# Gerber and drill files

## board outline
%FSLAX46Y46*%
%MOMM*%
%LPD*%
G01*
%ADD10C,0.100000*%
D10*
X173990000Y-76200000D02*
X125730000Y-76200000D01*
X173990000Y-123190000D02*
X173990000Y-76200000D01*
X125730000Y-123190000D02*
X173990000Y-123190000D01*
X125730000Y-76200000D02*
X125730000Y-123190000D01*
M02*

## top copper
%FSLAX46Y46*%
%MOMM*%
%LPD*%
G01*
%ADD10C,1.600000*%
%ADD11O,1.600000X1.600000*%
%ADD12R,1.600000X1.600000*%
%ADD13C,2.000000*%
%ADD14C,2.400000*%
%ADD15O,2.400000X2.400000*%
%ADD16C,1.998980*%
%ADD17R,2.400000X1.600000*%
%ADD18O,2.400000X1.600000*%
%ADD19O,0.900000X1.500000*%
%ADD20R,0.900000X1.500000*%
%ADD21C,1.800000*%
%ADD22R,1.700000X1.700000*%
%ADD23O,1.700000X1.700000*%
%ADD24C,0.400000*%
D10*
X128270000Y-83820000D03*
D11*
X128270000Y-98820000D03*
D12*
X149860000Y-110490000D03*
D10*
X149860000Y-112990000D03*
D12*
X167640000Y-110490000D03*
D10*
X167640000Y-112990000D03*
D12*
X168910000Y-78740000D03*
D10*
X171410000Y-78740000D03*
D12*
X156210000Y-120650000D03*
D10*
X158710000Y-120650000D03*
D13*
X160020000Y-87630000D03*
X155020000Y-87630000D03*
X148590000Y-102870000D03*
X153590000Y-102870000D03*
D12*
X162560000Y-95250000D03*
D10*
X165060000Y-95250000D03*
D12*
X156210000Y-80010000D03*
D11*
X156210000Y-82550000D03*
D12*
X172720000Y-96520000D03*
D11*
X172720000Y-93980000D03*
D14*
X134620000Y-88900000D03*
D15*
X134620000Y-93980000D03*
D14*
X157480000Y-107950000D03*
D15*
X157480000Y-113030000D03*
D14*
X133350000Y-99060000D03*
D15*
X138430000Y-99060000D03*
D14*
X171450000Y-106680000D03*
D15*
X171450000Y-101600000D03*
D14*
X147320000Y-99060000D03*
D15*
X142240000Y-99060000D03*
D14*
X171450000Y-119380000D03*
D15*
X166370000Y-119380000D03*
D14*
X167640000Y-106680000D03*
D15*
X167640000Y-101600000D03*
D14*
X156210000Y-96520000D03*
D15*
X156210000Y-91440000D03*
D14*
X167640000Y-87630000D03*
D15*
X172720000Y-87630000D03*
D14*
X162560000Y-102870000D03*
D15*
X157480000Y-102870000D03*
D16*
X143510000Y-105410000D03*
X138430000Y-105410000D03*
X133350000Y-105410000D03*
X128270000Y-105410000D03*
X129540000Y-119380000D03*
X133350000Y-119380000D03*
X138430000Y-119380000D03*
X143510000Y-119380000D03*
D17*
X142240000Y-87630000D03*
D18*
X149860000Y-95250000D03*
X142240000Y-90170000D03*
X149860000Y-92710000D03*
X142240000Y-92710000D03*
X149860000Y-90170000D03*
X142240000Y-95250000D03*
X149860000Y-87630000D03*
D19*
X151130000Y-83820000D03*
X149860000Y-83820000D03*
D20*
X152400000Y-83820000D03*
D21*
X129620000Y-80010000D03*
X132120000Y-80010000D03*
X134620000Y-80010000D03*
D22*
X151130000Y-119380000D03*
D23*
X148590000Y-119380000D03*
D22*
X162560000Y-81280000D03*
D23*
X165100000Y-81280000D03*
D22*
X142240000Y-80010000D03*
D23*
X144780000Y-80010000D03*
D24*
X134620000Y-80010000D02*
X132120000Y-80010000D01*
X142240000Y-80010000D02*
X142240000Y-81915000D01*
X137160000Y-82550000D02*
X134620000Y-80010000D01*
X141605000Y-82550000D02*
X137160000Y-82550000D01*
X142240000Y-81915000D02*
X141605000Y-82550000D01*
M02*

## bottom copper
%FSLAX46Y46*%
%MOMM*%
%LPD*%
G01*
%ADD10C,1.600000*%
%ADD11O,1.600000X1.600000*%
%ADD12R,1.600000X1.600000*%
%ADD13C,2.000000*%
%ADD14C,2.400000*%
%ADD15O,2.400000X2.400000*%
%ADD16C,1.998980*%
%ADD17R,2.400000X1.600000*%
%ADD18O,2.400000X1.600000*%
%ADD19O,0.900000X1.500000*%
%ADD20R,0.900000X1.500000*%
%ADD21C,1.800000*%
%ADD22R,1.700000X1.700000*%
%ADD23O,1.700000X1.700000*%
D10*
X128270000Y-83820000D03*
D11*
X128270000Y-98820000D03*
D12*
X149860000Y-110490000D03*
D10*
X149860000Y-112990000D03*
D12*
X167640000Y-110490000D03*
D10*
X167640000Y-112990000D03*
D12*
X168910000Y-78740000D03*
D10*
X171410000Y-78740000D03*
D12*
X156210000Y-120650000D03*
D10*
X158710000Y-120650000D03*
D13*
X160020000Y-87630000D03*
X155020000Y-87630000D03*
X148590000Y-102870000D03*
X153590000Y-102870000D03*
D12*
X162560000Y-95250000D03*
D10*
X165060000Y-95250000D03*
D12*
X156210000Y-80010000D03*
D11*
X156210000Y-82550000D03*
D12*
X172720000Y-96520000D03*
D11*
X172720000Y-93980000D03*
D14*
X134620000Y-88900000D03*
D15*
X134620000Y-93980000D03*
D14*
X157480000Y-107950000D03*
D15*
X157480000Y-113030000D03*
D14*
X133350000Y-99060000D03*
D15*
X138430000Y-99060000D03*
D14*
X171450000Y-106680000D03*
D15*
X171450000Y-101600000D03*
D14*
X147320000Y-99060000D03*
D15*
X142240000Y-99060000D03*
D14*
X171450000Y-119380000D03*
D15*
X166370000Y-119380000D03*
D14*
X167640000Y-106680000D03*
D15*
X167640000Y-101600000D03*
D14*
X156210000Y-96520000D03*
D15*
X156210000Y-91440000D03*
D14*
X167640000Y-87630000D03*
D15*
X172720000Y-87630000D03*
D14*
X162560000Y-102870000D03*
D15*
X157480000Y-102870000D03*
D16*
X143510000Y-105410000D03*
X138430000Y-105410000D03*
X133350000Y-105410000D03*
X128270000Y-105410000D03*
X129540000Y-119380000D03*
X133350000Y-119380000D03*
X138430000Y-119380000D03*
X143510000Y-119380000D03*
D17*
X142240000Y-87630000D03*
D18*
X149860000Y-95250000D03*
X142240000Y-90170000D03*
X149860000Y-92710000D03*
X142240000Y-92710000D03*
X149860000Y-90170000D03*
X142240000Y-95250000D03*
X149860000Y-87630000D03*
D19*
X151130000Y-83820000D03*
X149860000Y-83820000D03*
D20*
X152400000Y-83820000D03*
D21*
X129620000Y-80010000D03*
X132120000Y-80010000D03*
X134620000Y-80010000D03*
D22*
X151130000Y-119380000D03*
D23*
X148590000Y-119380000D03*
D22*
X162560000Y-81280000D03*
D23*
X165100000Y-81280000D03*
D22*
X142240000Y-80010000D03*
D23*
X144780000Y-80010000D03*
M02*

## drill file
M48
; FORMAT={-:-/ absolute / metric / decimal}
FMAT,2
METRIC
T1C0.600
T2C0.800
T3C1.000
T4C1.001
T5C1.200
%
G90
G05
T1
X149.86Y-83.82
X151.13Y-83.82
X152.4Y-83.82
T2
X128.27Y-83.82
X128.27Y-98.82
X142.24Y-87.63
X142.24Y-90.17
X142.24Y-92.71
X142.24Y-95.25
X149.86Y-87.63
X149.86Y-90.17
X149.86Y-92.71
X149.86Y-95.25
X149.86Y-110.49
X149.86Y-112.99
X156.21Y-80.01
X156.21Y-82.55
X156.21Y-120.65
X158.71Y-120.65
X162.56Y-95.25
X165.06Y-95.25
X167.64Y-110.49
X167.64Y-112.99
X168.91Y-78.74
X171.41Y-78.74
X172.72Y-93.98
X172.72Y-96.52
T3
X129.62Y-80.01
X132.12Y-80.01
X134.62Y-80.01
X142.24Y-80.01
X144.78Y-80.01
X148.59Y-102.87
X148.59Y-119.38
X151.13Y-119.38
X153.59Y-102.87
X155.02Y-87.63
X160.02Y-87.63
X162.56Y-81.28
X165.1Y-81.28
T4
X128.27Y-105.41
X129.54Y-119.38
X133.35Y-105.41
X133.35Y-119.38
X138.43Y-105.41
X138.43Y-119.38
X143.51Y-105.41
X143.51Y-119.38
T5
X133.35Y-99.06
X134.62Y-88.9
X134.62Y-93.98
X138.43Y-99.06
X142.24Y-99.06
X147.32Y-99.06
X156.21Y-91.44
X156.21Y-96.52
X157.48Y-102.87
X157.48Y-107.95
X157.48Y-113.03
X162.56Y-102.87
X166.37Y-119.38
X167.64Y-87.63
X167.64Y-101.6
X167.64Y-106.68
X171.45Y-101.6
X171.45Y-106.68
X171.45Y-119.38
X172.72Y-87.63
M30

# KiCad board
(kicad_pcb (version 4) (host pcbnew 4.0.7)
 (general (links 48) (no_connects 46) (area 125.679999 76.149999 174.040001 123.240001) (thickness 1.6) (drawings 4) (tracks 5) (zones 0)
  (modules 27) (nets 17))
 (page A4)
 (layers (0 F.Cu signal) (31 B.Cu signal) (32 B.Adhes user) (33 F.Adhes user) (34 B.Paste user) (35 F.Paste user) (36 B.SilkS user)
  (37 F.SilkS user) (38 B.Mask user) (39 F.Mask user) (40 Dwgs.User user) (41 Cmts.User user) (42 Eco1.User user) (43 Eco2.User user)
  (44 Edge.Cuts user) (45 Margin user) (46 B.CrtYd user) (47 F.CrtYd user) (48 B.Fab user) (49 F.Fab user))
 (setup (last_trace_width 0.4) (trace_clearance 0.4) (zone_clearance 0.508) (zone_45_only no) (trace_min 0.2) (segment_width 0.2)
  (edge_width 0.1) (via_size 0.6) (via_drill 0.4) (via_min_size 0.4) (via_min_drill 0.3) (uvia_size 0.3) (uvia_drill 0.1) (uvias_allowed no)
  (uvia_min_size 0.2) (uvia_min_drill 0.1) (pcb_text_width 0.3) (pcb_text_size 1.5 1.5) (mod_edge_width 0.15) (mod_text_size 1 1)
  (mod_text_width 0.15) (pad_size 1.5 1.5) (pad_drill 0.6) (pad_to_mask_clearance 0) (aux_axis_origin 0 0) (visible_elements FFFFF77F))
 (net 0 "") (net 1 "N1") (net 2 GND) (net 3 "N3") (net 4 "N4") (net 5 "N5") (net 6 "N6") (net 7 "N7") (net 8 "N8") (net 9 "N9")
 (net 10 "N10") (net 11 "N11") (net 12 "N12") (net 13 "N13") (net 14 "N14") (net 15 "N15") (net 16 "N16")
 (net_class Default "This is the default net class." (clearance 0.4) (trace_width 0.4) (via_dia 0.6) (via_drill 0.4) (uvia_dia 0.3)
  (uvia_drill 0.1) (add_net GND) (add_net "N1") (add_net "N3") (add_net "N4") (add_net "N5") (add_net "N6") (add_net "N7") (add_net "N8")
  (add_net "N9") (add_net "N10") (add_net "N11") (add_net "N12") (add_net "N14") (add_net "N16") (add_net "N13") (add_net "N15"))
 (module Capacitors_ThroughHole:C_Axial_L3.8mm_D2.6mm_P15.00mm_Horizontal (layer F.Cu) (at 128.27 83.82 270)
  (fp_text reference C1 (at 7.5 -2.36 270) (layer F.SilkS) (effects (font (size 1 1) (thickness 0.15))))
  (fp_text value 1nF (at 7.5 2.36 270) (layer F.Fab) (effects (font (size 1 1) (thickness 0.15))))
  (pad 1 thru_hole circle (at 0 0 270) (size 1.6 1.6) (drill 0.8) (layers *.Cu *.Mask) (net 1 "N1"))
  (pad 2 thru_hole oval (at 15 0 270) (size 1.6 1.6) (drill 0.8) (layers *.Cu *.Mask) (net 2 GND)))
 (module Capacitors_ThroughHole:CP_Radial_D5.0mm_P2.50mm (layer F.Cu) (at 149.86 110.49 270)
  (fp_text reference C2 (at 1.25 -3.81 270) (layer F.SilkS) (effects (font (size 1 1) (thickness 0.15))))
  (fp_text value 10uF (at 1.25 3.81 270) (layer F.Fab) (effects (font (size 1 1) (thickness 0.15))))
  (pad 1 thru_hole rect (at 0 0 270) (size 1.6 1.6) (drill 0.8) (layers *.Cu *.Mask) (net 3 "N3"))
  (pad 2 thru_hole circle (at 2.5 0 270) (size 1.6 1.6) (drill 0.8) (layers *.Cu *.Mask) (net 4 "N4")))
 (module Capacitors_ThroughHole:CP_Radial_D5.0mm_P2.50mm (layer F.Cu) (at 167.64 110.49 270)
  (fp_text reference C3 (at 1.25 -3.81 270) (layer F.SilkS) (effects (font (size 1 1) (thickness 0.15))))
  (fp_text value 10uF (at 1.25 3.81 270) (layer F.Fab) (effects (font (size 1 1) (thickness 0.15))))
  (pad 1 thru_hole rect (at 0 0 270) (size 1.6 1.6) (drill 0.8) (layers *.Cu *.Mask) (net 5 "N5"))
  (pad 2 thru_hole circle (at 2.5 0 270) (size 1.6 1.6) (drill 0.8) (layers *.Cu *.Mask) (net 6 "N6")))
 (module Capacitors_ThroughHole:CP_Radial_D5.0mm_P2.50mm (layer F.Cu) (at 168.91 78.74)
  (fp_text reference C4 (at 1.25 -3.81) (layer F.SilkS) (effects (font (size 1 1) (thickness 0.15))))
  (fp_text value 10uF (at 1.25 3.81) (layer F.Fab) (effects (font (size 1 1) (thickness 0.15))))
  (pad 1 thru_hole rect (at 0 0) (size 1.6 1.6) (drill 0.8) (layers *.Cu *.Mask) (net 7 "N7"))
  (pad 2 thru_hole circle (at 2.5 0) (size 1.6 1.6) (drill 0.8) (layers *.Cu *.Mask) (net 2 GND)))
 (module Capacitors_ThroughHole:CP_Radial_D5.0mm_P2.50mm (layer F.Cu) (at 156.21 120.65)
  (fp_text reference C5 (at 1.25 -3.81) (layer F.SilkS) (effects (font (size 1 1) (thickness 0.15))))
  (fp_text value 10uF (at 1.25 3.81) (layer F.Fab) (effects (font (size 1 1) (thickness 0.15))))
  (pad 1 thru_hole rect (at 0 0) (size 1.6 1.6) (drill 0.8) (layers *.Cu *.Mask) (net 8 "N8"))
  (pad 2 thru_hole circle (at 2.5 0) (size 1.6 1.6) (drill 0.8) (layers *.Cu *.Mask) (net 2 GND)))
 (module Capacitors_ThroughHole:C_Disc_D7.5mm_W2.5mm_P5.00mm (layer F.Cu) (at 160.02 87.63 180)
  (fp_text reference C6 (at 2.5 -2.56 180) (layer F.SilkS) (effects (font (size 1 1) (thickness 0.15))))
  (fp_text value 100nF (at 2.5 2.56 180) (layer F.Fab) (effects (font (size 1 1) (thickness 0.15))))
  (pad 1 thru_hole circle (at 0 0 180) (size 2 2) (drill 1) (layers *.Cu *.Mask) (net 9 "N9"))
  (pad 2 thru_hole circle (at 5 0 180) (size 2 2) (drill 1) (layers *.Cu *.Mask) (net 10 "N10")))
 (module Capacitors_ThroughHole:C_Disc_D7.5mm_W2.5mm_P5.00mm (layer F.Cu) (at 148.59 102.87)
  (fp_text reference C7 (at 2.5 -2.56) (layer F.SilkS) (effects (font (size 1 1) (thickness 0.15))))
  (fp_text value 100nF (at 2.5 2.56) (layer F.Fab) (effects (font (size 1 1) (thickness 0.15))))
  (pad 1 thru_hole circle (at 0 0) (size 2 2) (drill 1) (layers *.Cu *.Mask) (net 2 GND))
  (pad 2 thru_hole circle (at 5 0) (size 2 2) (drill 1) (layers *.Cu *.Mask) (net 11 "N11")))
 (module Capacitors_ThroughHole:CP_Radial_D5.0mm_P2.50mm (layer F.Cu) (at 162.56 95.25)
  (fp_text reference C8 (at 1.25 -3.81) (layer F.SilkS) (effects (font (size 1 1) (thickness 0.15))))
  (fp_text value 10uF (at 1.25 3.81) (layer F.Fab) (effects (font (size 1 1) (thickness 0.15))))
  (pad 1 thru_hole rect (at 0 0) (size 1.6 1.6) (drill 0.8) (layers *.Cu *.Mask) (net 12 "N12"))
  (pad 2 thru_hole circle (at 2.5 0) (size 1.6 1.6) (drill 0.8) (layers *.Cu *.Mask) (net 2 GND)))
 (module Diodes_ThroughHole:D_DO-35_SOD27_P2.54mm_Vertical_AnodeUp (layer F.Cu) (at 156.21 80.01 270)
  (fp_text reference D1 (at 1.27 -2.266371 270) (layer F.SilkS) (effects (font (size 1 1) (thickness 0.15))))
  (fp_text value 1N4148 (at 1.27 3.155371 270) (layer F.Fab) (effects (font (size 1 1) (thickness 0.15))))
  (pad 1 thru_hole rect (at 0 0 270) (size 1.6 1.6) (drill 0.8) (layers *.Cu *.Mask) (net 9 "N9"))
  (pad 2 thru_hole oval (at 2.54 0 270) (size 1.6 1.6) (drill 0.8) (layers *.Cu *.Mask) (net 2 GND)))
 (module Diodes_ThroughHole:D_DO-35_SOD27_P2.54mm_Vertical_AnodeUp (layer F.Cu) (at 172.72 96.52 90)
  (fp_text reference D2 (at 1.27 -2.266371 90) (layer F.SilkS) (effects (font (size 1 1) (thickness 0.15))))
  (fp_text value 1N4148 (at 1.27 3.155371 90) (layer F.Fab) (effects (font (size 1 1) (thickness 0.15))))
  (pad 1 thru_hole rect (at 0 0 90) (size 1.6 1.6) (drill 0.8) (layers *.Cu *.Mask) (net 11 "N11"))
  (pad 2 thru_hole oval (at 2.54 0 90) (size 1.6 1.6) (drill 0.8) (layers *.Cu *.Mask) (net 9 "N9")))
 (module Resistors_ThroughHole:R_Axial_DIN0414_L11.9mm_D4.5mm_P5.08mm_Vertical (layer F.Cu) (at 134.62 88.9 270)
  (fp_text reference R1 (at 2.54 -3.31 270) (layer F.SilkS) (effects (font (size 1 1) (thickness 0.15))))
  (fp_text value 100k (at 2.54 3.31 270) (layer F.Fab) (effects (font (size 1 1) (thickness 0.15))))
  (pad 1 thru_hole circle (at 0 0 270) (size 2.4 2.4) (drill 1.2) (layers *.Cu *.Mask) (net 8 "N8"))
  (pad 2 thru_hole oval (at 5.08 0 270) (size 2.4 2.4) (drill 1.2) (layers *.Cu *.Mask) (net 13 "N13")))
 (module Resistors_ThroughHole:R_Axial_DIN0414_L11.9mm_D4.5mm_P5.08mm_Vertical (layer F.Cu) (at 157.48 107.95 270)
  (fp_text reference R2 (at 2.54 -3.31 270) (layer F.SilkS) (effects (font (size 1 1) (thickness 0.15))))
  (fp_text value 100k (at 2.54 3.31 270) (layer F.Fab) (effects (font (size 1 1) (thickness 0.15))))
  (pad 1 thru_hole circle (at 0 0 270) (size 2.4 2.4) (drill 1.2) (layers *.Cu *.Mask) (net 13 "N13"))
  (pad 2 thru_hole oval (at 5.08 0 270) (size 2.4 2.4) (drill 1.2) (layers *.Cu *.Mask) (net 2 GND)))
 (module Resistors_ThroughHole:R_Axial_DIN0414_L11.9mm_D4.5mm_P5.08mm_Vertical (layer F.Cu) (at 133.35 99.06)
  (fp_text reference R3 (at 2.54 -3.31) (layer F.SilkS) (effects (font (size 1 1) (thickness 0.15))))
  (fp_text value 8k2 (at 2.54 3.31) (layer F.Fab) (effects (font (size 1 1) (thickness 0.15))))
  (pad 1 thru_hole circle (at 0 0) (size 2.4 2.4) (drill 1.2) (layers *.Cu *.Mask) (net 3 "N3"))
  (pad 2 thru_hole oval (at 5.08 0) (size 2.4 2.4) (drill 1.2) (layers *.Cu *.Mask) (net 1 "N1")))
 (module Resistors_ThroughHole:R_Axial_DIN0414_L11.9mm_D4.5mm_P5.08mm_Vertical (layer F.Cu) (at 171.45 106.68 90)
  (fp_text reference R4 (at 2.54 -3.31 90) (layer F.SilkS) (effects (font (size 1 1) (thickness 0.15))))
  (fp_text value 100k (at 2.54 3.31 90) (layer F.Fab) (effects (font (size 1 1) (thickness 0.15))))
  (pad 1 thru_hole circle (at 0 0 90) (size 2.4 2.4) (drill 1.2) (layers *.Cu *.Mask) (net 3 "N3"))
  (pad 2 thru_hole oval (at 5.08 0 90) (size 2.4 2.4) (drill 1.2) (layers *.Cu *.Mask) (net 13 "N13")))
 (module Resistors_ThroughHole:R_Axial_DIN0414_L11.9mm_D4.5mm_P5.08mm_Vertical (layer F.Cu) (at 147.32 99.06 180)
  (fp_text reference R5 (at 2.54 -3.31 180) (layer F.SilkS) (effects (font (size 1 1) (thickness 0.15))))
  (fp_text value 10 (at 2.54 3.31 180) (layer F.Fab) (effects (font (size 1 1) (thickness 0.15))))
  (pad 1 thru_hole circle (at 0 0 180) (size 2.4 2.4) (drill 1.2) (layers *.Cu *.Mask) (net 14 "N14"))
  (pad 2 thru_hole oval (at 5.08 0 180) (size 2.4 2.4) (drill 1.2) (layers *.Cu *.Mask) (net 2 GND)))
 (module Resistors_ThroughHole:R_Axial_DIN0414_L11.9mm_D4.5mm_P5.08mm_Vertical (layer F.Cu) (at 171.45 119.38 180)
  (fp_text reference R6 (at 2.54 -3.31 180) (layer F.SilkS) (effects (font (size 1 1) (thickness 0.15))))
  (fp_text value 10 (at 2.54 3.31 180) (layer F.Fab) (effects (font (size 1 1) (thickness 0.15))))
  (pad 1 thru_hole circle (at 0 0 180) (size 2.4 2.4) (drill 1.2) (layers *.Cu *.Mask) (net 6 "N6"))
  (pad 2 thru_hole oval (at 5.08 0 180) (size 2.4 2.4) (drill 1.2) (layers *.Cu *.Mask) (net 2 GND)))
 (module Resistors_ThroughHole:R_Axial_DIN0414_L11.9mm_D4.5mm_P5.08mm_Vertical (layer F.Cu) (at 167.64 106.68 90)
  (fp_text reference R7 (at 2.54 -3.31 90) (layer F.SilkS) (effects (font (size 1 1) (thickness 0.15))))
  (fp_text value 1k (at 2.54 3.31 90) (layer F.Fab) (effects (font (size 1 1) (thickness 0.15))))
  (pad 1 thru_hole circle (at 0 0 90) (size 2.4 2.4) (drill 1.2) (layers *.Cu *.Mask) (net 5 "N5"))
  (pad 2 thru_hole oval (at 5.08 0 90) (size 2.4 2.4) (drill 1.2) (layers *.Cu *.Mask) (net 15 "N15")))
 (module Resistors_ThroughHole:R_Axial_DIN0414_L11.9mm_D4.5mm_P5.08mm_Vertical (layer F.Cu) (at 156.21 96.52 90)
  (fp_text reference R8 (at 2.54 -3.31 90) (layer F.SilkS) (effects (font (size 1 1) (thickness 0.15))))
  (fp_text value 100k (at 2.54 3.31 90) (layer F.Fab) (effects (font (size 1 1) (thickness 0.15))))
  (pad 1 thru_hole circle (at 0 0 90) (size 2.4 2.4) (drill 1.2) (layers *.Cu *.Mask) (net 8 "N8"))
  (pad 2 thru_hole oval (at 5.08 0 90) (size 2.4 2.4) (drill 1.2) (layers *.Cu *.Mask) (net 7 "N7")))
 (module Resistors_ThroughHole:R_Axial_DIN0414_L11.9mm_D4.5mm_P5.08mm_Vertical (layer F.Cu) (at 167.64 87.63)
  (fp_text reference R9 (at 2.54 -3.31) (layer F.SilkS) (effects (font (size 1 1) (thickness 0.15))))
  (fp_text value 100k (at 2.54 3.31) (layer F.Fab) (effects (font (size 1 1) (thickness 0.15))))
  (pad 1 thru_hole circle (at 0 0) (size 2.4 2.4) (drill 1.2) (layers *.Cu *.Mask) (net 7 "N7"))
  (pad 2 thru_hole oval (at 5.08 0) (size 2.4 2.4) (drill 1.2) (layers *.Cu *.Mask) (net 2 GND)))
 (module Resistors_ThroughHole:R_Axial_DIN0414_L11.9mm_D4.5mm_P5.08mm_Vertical (layer F.Cu) (at 162.56 102.87 180)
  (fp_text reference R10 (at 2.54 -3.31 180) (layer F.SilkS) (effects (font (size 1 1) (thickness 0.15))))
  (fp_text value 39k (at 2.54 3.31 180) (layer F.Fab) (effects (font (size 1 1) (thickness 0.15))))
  (pad 1 thru_hole circle (at 0 0 180) (size 2.4 2.4) (drill 1.2) (layers *.Cu *.Mask) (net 15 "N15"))
  (pad 2 thru_hole oval (at 5.08 0 180) (size 2.4 2.4) (drill 1.2) (layers *.Cu *.Mask) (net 10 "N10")))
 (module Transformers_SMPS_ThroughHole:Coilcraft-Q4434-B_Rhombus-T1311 (layer F.Cu) (at 135.89 113.03)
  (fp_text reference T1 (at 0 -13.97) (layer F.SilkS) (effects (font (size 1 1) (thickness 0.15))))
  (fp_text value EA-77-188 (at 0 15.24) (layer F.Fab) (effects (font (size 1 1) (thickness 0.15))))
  (pad 5 thru_hole circle (at 7.62 -7.62) (size 1.99898 1.99898) (drill 1.00076) (layers *.Cu *.Mask))
  (pad 6 thru_hole circle (at 2.54 -7.62) (size 1.99898 1.99898) (drill 1.00076) (layers *.Cu *.Mask))
  (pad 7 thru_hole circle (at -2.54 -7.62) (size 1.99898 1.99898) (drill 1.00076) (layers *.Cu *.Mask))
  (pad 8 thru_hole circle (at -7.62 -7.62) (size 1.99898 1.99898) (drill 1.00076) (layers *.Cu *.Mask))
  (pad 1 thru_hole circle (at -6.35 6.35) (size 1.99898 1.99898) (drill 1.00076) (layers *.Cu *.Mask) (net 4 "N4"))
  (pad 2 thru_hole circle (at -2.54 6.35) (size 1.99898 1.99898) (drill 1.00076) (layers *.Cu *.Mask) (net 2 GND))
  (pad 3 thru_hole circle (at 2.54 6.35) (size 1.99898 1.99898) (drill 1.00076) (layers *.Cu *.Mask) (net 2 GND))
  (pad 4 thru_hole circle (at 7.62 6.35) (size 1.99898 1.99898) (drill 1.00076) (layers *.Cu *.Mask) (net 14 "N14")))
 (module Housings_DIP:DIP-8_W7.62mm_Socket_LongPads (layer F.Cu) (at 142.24 87.63)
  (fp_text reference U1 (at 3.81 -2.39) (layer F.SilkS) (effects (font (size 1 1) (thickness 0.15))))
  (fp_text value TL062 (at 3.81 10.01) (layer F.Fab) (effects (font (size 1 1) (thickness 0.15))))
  (pad 1 thru_hole rect (at 0 0) (size 2.4 1.6) (drill 0.8) (layers *.Cu *.Mask) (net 3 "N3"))
  (pad 5 thru_hole oval (at 7.62 7.62) (size 2.4 1.6) (drill 0.8) (layers *.Cu *.Mask) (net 7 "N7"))
  (pad 2 thru_hole oval (at 0 2.54) (size 2.4 1.6) (drill 0.8) (layers *.Cu *.Mask) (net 1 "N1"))
  (pad 6 thru_hole oval (at 7.62 5.08) (size 2.4 1.6) (drill 0.8) (layers *.Cu *.Mask) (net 15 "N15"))
  (pad 3 thru_hole oval (at 0 5.08) (size 2.4 1.6) (drill 0.8) (layers *.Cu *.Mask) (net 13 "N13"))
  (pad 7 thru_hole oval (at 7.62 2.54) (size 2.4 1.6) (drill 0.8) (layers *.Cu *.Mask) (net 10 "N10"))
  (pad 4 thru_hole oval (at 0 7.62) (size 2.4 1.6) (drill 0.8) (layers *.Cu *.Mask) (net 2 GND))
  (pad 8 thru_hole oval (at 7.62 0) (size 2.4 1.6) (drill 0.8) (layers *.Cu *.Mask) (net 8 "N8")))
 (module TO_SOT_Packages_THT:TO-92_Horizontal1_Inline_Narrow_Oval (layer F.Cu) (at 152.4 83.82 180)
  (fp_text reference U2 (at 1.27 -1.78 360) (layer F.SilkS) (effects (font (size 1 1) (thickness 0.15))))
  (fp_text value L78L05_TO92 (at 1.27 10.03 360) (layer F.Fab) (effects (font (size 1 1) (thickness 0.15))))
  (pad 2 thru_hole oval (at 1.27 0) (size 0.9 1.5) (drill 0.6) (layers *.Cu *.Mask) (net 2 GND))
  (pad 3 thru_hole oval (at 2.54 0) (size 0.9 1.5) (drill 0.6) (layers *.Cu *.Mask) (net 12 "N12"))
  (pad 1 thru_hole rect (at 0 0) (size 0.9 1.5) (drill 0.6) (layers *.Cu *.Mask) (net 8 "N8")))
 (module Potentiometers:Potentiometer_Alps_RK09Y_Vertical (layer F.Cu) (at 134.62 80.01 90)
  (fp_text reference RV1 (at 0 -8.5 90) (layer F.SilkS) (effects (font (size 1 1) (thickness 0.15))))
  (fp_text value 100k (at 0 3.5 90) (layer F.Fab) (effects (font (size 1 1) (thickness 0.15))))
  (pad 3 thru_hole circle (at 0 -5 90) (size 1.8 1.8) (drill 1) (layers *.Cu *.Mask) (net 11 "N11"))
  (pad 2 thru_hole circle (at 0 -2.5 90) (size 1.8 1.8) (drill 1) (layers *.Cu *.Mask) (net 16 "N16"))
  (pad 1 thru_hole circle (at 0 0 90) (size 1.8 1.8) (drill 1) (layers *.Cu *.Mask) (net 16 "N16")))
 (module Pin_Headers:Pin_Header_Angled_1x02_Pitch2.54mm (layer F.Cu) (at 151.13 119.38 270)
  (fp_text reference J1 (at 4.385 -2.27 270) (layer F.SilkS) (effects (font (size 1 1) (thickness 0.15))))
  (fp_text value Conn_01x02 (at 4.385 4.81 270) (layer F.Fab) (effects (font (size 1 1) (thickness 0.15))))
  (pad 1 thru_hole rect (at 0 0 270) (size 1.7 1.7) (drill 1) (layers *.Cu *.Mask) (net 14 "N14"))
  (pad 2 thru_hole oval (at 0 2.54 270) (size 1.7 1.7) (drill 1) (layers *.Cu *.Mask) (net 6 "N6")))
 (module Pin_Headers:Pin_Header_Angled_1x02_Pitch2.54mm (layer F.Cu) (at 162.56 81.28 90)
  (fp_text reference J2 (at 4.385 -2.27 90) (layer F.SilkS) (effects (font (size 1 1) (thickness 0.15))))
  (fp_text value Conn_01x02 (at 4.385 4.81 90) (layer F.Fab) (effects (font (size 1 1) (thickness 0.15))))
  (pad 1 thru_hole rect (at 0 0 90) (size 1.7 1.7) (drill 1) (layers *.Cu *.Mask) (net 12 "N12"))
  (pad 2 thru_hole oval (at 0 2.54 90) (size 1.7 1.7) (drill 1) (layers *.Cu *.Mask) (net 2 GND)))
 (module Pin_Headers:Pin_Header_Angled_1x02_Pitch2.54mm (layer F.Cu) (at 142.24 80.01 90)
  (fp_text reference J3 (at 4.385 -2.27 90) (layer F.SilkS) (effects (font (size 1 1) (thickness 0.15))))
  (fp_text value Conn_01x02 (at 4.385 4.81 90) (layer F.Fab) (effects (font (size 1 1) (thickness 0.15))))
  (pad 1 thru_hole rect (at 0 0 90) (size 1.7 1.7) (drill 1) (layers *.Cu *.Mask) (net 16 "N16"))
  (pad 2 thru_hole oval (at 0 2.54 90) (size 1.7 1.7) (drill 1) (layers *.Cu *.Mask) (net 2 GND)))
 (gr_line (start 173.99 76.2) (end 125.73 76.2) (angle 90) (layer Edge.Cuts) (width 0.1))
 (gr_line (start 173.99 123.19) (end 173.99 76.2) (angle 90) (layer Edge.Cuts) (width 0.1))
 (gr_line (start 125.73 123.19) (end 173.99 123.19) (angle 90) (layer Edge.Cuts) (width 0.1))
 (gr_line (start 125.73 76.2) (end 125.73 123.19) (angle 90) (layer Edge.Cuts) (width 0.1))
 (segment (start 134.62 80.01) (end 132.12 80.01) (width 0.4) (layer F.Cu) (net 16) (status C00000))
 (segment (start 142.24 80.01) (end 142.24 81.915) (width 0.4) (layer F.Cu) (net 16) (status 400000))
 (segment (start 137.16 82.55) (end 134.62 80.01) (width 0.4) (layer F.Cu) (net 16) (status 800000))
 (segment (start 141.605 82.55) (end 137.16 82.55) (width 0.4) (layer F.Cu) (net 16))
 (segment (start 142.24 81.915) (end 141.605 82.55) (width 0.4) (layer F.Cu) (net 16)))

